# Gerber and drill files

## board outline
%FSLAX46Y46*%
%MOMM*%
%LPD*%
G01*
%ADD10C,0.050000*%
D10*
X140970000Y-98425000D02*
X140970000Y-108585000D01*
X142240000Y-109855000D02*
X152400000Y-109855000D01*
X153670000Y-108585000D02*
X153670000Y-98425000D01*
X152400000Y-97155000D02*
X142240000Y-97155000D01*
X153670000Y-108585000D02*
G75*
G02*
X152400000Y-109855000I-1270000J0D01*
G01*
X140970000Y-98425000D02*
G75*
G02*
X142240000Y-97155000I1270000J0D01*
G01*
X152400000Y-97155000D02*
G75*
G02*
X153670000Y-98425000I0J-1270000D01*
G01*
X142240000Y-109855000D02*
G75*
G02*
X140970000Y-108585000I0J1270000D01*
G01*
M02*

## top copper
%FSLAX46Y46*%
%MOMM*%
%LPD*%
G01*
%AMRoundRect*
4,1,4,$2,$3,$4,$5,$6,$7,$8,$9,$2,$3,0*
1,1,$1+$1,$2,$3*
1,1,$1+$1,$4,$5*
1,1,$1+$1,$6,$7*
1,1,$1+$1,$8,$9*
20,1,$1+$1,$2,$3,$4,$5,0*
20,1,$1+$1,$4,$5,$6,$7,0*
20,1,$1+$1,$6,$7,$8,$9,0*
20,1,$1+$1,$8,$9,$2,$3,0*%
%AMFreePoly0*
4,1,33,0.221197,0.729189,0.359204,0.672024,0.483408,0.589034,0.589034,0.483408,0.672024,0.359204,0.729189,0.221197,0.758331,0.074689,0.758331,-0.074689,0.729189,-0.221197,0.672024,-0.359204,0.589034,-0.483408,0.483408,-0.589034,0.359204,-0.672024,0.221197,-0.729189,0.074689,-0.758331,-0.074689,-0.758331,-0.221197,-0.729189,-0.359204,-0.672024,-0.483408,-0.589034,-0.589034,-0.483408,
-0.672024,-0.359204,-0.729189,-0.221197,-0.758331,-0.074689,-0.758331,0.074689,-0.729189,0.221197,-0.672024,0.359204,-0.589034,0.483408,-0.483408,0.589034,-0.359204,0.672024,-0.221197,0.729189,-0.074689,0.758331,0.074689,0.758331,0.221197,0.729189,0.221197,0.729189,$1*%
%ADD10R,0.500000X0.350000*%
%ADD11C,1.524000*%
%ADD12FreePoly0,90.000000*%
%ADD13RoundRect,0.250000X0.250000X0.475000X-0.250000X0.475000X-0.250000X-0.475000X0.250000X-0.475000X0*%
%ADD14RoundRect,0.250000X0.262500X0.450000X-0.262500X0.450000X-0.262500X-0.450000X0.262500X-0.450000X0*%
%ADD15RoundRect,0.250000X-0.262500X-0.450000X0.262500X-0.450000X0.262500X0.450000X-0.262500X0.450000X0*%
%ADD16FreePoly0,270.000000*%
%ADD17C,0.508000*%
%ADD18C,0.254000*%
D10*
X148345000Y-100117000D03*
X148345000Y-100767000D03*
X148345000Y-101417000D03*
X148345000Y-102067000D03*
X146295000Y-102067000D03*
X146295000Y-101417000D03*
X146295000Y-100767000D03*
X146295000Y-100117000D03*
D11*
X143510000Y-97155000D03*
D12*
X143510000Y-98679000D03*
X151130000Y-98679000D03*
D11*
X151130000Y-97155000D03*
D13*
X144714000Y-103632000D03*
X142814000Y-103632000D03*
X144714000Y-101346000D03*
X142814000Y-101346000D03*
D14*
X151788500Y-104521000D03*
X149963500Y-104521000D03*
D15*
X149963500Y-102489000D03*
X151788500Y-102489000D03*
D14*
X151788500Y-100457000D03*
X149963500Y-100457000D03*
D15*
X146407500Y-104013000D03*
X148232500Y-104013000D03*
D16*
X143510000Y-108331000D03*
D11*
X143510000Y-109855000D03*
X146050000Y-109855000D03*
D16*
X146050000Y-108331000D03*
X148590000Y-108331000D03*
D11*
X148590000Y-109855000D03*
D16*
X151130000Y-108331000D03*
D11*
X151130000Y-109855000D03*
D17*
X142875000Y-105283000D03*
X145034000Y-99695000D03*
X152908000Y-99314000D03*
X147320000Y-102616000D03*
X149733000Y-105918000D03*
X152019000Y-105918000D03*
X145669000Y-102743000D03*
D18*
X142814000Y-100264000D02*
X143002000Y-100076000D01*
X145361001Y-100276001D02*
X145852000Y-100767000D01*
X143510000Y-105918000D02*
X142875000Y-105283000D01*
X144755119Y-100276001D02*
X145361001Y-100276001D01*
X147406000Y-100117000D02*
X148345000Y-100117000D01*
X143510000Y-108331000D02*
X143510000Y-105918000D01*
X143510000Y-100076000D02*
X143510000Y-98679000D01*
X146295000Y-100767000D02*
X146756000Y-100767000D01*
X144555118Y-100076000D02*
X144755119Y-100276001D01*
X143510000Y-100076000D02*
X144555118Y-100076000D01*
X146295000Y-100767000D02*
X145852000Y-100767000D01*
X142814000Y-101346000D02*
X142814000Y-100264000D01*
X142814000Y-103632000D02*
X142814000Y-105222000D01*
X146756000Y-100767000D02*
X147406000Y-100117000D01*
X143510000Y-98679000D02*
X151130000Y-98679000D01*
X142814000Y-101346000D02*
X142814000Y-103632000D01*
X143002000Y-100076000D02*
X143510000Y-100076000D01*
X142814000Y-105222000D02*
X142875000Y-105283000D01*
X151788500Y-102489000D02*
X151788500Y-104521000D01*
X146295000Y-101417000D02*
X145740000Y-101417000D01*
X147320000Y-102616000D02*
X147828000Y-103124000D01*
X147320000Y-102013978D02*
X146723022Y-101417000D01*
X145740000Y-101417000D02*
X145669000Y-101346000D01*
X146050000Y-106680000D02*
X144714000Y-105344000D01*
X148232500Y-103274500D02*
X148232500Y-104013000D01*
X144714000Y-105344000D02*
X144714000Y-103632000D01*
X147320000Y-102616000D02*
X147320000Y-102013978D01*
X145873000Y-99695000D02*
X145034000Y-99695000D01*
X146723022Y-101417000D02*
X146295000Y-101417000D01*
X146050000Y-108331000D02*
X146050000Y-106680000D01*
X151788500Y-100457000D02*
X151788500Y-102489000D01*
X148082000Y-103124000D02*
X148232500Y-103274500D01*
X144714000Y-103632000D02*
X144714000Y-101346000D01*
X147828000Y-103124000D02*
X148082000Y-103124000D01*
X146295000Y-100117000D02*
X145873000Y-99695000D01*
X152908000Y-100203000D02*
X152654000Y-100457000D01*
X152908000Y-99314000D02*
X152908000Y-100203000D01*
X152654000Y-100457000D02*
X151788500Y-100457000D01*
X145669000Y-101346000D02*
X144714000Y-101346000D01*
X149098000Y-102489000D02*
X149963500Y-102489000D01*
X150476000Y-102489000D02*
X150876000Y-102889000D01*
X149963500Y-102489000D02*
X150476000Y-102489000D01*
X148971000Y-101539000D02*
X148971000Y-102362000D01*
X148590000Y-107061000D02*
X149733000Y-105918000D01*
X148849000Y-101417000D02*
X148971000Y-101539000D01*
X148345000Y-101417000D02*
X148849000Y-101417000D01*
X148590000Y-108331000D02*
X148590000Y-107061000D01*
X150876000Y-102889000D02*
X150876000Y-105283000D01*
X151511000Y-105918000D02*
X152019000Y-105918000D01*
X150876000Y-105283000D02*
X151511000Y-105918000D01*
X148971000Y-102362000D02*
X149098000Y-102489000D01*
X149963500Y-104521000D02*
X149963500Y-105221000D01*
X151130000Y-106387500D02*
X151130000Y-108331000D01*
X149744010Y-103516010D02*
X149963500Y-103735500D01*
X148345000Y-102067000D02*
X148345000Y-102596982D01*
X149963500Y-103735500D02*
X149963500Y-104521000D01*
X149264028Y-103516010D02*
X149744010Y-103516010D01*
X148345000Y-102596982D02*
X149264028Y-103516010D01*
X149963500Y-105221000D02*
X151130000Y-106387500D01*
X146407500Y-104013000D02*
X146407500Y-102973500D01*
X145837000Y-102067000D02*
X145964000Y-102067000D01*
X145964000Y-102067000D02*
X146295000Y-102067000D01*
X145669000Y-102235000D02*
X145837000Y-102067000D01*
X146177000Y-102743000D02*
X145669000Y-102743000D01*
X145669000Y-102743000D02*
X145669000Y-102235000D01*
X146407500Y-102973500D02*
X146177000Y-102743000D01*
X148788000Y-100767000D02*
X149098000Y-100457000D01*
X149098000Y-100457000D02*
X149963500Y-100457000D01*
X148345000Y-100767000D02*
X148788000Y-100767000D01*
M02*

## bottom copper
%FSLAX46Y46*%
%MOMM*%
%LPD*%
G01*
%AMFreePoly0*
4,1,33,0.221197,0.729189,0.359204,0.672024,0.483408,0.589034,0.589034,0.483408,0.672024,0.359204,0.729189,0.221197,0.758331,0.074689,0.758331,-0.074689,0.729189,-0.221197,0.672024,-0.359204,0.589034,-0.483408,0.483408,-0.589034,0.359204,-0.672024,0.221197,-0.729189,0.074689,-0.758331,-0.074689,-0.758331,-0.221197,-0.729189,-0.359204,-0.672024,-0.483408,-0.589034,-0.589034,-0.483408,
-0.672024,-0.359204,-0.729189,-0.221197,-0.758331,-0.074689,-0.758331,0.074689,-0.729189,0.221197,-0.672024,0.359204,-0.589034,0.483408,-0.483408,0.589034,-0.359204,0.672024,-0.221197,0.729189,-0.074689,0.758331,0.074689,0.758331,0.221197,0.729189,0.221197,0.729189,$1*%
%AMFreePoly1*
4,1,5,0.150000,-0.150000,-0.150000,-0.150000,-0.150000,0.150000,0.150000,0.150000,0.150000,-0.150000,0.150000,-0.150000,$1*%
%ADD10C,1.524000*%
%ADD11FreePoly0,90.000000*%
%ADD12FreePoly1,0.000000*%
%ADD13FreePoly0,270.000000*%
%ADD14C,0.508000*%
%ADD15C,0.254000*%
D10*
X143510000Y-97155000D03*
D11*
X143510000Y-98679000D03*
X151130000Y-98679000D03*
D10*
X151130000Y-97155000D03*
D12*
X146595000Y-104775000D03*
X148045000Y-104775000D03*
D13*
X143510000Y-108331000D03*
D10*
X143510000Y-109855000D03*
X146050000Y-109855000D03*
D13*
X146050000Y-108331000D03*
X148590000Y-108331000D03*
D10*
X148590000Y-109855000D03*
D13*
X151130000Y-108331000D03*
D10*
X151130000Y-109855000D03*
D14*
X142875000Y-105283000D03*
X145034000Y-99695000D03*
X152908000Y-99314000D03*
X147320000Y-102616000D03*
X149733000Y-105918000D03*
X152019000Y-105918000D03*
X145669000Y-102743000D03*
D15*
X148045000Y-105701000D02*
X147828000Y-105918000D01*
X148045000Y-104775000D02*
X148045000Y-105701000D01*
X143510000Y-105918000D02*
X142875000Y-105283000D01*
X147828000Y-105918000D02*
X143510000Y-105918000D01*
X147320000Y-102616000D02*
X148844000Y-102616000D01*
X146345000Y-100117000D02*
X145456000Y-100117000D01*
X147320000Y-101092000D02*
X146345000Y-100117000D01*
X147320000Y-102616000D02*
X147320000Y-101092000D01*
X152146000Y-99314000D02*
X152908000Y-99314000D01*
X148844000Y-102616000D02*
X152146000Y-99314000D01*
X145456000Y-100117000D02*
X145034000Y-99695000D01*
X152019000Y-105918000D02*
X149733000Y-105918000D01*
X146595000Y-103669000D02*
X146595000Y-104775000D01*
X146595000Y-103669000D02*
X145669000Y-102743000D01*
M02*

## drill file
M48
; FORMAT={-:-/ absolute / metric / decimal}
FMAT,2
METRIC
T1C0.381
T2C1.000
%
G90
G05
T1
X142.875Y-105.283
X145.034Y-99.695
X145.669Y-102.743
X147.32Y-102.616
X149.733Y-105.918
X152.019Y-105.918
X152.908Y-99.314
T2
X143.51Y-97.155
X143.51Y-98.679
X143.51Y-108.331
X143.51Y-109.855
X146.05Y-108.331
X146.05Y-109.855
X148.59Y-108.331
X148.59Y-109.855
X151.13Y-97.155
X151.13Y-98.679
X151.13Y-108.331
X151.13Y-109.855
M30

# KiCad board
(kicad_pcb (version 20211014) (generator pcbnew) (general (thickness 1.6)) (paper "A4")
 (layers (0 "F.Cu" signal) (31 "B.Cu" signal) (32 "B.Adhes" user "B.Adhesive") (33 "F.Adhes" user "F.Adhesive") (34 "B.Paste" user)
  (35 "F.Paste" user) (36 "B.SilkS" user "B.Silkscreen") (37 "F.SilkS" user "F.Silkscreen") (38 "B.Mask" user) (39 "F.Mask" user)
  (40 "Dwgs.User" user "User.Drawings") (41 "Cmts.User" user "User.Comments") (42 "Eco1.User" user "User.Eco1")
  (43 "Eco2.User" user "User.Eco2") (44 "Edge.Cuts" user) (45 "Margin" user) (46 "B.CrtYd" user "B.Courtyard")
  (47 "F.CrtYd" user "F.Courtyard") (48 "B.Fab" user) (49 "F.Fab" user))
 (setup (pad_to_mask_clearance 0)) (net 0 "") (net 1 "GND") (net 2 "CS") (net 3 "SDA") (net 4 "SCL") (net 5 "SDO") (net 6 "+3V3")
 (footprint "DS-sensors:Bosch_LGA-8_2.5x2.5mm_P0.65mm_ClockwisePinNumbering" (layer "F.Cu") (at 147.32 101.092 -90)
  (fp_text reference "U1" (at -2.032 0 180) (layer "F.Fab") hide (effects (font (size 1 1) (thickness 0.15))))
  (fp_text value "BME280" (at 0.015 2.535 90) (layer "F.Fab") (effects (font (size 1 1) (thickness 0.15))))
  (pad "1" smd rect locked (at -0.975 -1.025) (size 0.5 0.35) (layers "F.Cu" "F.Paste" "F.Mask") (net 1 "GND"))
  (pad "2" smd rect locked (at -0.325 -1.025) (size 0.5 0.35) (layers "F.Cu" "F.Paste" "F.Mask") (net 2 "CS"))
  (pad "3" smd rect locked (at 0.325 -1.025) (size 0.5 0.35) (layers "F.Cu" "F.Paste" "F.Mask") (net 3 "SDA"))
  (pad "4" smd rect locked (at 0.975 -1.025) (size 0.5 0.35) (layers "F.Cu" "F.Paste" "F.Mask") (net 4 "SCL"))
  (pad "5" smd rect locked (at 0.975 1.025) (size 0.5 0.35) (layers "F.Cu" "F.Paste" "F.Mask") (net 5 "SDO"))
  (pad "6" smd rect locked (at 0.325 1.025) (size 0.5 0.35) (layers "F.Cu" "F.Paste" "F.Mask") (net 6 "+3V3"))
  (pad "7" smd rect locked (at -0.325 1.025) (size 0.5 0.35) (layers "F.Cu" "F.Paste" "F.Mask") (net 1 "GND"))
  (pad "8" smd rect locked (at -0.975 1.025) (size 0.5 0.35) (layers "F.Cu" "F.Paste" "F.Mask") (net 6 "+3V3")))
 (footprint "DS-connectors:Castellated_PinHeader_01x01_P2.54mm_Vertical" (layer "F.Cu") (at 141.478 98.679 90)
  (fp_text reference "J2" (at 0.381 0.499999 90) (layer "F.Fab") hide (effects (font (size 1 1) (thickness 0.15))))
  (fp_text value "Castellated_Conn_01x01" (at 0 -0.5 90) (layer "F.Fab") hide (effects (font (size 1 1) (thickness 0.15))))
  (pad "1" thru_hole circle locked (at 1.524 2.032 90) (size 1.524 1.524) (drill 1) (layers *.Cu *.Mask) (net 1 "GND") (zone_connect 0))
  (pad "1" thru_hole custom locked (at 0 2.032 90) (size 1.524 1.524) (drill 1) (layers *.Cu *.Mask) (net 1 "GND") (zone_connect 0)
   (options (clearance outline) (anchor circle)) (primitives)))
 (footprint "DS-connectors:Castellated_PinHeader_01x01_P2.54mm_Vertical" (layer "F.Cu") (at 149.098 98.679 90)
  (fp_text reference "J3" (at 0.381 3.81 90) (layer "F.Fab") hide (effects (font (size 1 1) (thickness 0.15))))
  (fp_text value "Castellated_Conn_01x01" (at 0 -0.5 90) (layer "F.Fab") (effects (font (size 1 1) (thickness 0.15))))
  (pad "1" thru_hole custom locked (at 0 2.032 90) (size 1.524 1.524) (drill 1) (layers *.Cu *.Mask) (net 1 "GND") (zone_connect 0)
   (options (clearance outline) (anchor circle)) (primitives))
  (pad "1" thru_hole circle locked (at 1.524 2.032 90) (size 1.524 1.524) (drill 1) (layers *.Cu *.Mask) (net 1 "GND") (zone_connect 0)))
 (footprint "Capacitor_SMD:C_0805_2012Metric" (layer "F.Cu") (at 143.764 103.632 180)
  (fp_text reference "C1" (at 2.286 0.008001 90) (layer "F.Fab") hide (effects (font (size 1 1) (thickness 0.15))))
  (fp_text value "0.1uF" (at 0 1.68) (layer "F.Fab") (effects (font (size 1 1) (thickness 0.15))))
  (pad "1" smd roundrect locked (at -0.95 0 180) (size 1 1.45) (layers "F.Cu" "F.Paste" "F.Mask") (roundrect_rratio 0.25) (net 6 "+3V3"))
  (pad "2" smd roundrect locked (at 0.95 0 180) (size 1 1.45) (layers "F.Cu" "F.Paste" "F.Mask") (roundrect_rratio 0.25) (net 1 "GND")))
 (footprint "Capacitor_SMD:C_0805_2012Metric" (layer "F.Cu") (at 143.764 101.346 180)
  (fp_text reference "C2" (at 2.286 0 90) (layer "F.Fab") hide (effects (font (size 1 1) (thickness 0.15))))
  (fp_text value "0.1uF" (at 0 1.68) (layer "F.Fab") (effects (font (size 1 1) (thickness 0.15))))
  (pad "1" smd roundrect locked (at -0.95 0 180) (size 1 1.45) (layers "F.Cu" "F.Paste" "F.Mask") (roundrect_rratio 0.25) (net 6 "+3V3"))
  (pad "2" smd roundrect locked (at 0.95 0 180) (size 1 1.45) (layers "F.Cu" "F.Paste" "F.Mask") (roundrect_rratio 0.25) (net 1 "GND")))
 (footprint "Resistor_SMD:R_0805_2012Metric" (layer "F.Cu") (at 150.876 104.521 180)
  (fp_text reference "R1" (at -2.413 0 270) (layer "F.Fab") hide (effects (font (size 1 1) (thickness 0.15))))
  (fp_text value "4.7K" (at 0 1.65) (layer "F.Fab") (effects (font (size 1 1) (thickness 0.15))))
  (pad "1" smd roundrect locked (at -0.9125 0 180) (size 1.025 1.4) (layers "F.Cu" "F.Paste" "F.Mask") (roundrect_rratio 0.243902)
   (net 6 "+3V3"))
  (pad "2" smd roundrect locked (at 0.9125 0 180) (size 1.025 1.4) (layers "F.Cu" "F.Paste" "F.Mask") (roundrect_rratio 0.243902)
   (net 4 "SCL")))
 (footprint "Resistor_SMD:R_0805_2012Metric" (layer "F.Cu") (at 150.876 102.489)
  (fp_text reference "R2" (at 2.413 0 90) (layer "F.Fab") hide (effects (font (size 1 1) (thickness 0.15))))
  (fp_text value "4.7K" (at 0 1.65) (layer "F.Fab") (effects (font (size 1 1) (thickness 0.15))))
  (pad "1" smd roundrect locked (at -0.9125 0) (size 1.025 1.4) (layers "F.Cu" "F.Paste" "F.Mask") (roundrect_rratio 0.243902) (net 3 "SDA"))
  (pad "2" smd roundrect locked (at 0.9125 0) (size 1.025 1.4) (layers "F.Cu" "F.Paste" "F.Mask") (roundrect_rratio 0.243902) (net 6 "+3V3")))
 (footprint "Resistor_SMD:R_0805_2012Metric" (layer "F.Cu") (at 150.876 100.457 180)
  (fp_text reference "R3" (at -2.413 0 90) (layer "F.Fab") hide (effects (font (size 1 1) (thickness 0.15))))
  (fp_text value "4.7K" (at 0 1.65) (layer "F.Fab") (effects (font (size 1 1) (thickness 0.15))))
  (pad "1" smd roundrect locked (at -0.9125 0 180) (size 1.025 1.4) (layers "F.Cu" "F.Paste" "F.Mask") (roundrect_rratio 0.243902)
   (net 6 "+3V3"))
  (pad "2" smd roundrect locked (at 0.9125 0 180) (size 1.025 1.4) (layers "F.Cu" "F.Paste" "F.Mask") (roundrect_rratio 0.243902)
   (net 2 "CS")))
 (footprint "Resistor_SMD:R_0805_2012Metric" (layer "F.Cu") (at 147.32 104.013)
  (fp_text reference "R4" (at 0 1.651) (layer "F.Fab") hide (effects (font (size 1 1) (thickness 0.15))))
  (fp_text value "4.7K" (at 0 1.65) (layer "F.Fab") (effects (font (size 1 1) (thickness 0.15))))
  (pad "1" smd roundrect locked (at -0.9125 0) (size 1.025 1.4) (layers "F.Cu" "F.Paste" "F.Mask") (roundrect_rratio 0.243902) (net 5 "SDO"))
  (pad "2" smd roundrect locked (at 0.9125 0) (size 1.025 1.4) (layers "F.Cu" "F.Paste" "F.Mask") (roundrect_rratio 0.243902) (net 6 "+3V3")))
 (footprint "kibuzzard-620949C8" (layer "F.Cu") (at 143.51 105.537 90)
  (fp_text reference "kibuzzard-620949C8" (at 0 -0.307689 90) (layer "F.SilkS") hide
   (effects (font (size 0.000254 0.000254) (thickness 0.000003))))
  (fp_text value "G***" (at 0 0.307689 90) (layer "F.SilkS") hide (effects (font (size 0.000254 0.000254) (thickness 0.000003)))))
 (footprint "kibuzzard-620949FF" (layer "F.Cu") (at 151.13 107.061 90)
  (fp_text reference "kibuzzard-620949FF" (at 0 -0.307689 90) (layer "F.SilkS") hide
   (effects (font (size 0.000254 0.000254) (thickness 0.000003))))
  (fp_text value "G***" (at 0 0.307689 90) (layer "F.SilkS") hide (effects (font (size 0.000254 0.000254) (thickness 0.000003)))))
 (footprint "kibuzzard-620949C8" (layer "F.Cu") (at 148.59 106.299 90)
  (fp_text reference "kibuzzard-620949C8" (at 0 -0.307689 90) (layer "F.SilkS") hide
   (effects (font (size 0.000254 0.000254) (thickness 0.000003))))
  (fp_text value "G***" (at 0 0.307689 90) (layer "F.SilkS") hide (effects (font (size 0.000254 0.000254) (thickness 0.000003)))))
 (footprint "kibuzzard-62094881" (layer "F.Cu") (at 148.717 97.917)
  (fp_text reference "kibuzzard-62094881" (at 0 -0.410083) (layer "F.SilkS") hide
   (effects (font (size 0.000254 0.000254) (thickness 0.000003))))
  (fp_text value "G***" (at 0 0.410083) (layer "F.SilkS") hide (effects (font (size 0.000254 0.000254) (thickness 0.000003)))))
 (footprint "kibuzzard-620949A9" (layer "F.Cu") (at 143.51 107.061 90)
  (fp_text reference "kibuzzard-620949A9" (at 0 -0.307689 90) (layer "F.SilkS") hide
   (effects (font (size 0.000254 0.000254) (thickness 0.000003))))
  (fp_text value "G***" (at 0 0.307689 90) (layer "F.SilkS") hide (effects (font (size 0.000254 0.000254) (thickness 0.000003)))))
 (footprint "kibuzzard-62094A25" (layer "F.Cu") (at 151.13 106.299 90)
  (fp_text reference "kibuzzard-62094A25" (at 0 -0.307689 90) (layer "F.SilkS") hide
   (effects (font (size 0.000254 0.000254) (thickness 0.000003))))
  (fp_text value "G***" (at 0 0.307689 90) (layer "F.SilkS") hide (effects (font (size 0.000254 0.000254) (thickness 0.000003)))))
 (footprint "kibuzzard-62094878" (layer "F.Cu") (at 147.7772 97.917)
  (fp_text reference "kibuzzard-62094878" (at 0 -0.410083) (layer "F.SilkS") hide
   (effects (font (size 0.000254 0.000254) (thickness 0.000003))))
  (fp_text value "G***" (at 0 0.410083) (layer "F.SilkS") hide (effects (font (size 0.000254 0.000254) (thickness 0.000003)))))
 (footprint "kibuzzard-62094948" (layer "F.Cu") (at 147.32 98.933)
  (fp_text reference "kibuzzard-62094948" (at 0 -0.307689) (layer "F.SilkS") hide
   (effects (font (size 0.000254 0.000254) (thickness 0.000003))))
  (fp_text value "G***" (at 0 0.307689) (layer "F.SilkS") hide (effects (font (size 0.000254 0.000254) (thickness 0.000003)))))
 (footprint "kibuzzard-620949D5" (layer "F.Cu") (at 146.05 105.537 90)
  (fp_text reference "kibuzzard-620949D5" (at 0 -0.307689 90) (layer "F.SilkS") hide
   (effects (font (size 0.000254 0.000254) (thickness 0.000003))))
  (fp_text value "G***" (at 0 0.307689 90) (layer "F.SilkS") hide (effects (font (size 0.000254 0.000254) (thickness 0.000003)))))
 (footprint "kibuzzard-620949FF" (layer "F.Cu") (at 148.59 107.061 90)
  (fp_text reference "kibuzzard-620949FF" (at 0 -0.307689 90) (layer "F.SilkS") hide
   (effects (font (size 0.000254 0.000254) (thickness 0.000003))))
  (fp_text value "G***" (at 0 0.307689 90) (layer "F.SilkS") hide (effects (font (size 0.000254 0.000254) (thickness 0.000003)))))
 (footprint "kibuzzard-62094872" (layer "F.Cu") (at 146.9136 97.917)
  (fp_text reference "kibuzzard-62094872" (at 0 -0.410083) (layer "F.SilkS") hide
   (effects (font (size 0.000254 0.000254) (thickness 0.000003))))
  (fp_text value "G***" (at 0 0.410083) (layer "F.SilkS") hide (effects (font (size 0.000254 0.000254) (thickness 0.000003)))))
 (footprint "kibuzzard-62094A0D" (layer "F.Cu") (at 148.59 105.537 90)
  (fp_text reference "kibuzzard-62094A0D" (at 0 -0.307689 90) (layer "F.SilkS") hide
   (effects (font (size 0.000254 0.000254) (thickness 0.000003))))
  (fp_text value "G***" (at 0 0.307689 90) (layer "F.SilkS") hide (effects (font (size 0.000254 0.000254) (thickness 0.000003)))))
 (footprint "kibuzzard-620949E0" (layer "F.Cu") (at 146.05 106.299 90)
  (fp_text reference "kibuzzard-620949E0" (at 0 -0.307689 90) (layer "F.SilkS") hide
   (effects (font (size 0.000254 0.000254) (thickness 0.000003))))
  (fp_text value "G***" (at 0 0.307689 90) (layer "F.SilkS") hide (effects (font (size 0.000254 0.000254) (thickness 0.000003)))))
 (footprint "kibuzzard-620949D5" (layer "F.Cu") (at 146.05 107.061 90)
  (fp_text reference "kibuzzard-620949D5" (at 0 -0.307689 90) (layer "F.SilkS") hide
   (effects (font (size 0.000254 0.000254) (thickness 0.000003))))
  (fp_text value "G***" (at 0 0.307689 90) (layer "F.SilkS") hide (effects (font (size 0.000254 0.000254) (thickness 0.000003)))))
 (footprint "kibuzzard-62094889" (layer "F.Cu") (at 149.6568 97.917)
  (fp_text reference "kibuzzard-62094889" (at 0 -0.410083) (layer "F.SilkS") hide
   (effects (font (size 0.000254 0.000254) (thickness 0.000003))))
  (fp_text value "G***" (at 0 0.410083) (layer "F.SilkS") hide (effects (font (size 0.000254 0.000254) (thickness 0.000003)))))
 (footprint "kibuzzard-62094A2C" (layer "F.Cu") (at 151.13 105.537 90)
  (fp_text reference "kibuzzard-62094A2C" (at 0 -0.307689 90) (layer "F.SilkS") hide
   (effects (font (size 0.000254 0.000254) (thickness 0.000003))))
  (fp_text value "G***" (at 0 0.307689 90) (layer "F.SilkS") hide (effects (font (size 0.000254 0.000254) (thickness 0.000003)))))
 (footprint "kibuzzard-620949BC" (layer "F.Cu") (at 143.51 106.299 90)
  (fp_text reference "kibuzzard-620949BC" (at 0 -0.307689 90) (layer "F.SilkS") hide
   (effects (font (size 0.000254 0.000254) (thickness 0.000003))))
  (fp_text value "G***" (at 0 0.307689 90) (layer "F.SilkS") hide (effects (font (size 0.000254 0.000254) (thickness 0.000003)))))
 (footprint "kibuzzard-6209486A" (layer "F.Cu") (at 145.9484 97.917)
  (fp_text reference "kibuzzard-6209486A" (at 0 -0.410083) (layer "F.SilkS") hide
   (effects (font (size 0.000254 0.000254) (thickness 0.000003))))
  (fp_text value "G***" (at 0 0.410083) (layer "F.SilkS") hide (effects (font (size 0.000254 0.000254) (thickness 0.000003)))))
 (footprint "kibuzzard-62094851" (layer "F.Cu") (at 144.9324 97.917)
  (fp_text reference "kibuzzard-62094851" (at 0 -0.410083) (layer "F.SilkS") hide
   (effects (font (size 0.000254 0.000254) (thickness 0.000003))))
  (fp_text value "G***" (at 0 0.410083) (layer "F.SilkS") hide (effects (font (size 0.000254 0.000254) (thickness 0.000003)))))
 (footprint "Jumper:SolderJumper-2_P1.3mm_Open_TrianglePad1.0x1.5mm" (layer "B.Cu") (at 147.32 104.775)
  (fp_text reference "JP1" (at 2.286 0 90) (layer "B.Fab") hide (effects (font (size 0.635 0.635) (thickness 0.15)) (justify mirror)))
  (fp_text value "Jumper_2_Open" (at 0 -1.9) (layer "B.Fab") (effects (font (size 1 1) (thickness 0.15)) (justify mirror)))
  (pad "1" smd custom locked (at -0.725 0) (size 0.3 0.3) (layers "B.Cu" "B.Mask") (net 5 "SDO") (zone_connect 2)
   (options (clearance outline) (anchor rect)) (primitives))
  (pad "2" smd custom locked (at 0.725 0) (size 0.3 0.3) (layers "B.Cu" "B.Mask") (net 1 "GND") (zone_connect 2)
   (options (clearance outline) (anchor rect)) (primitives)))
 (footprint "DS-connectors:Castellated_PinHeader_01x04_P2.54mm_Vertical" (layer "B.Cu") (at 140.97 108.331 -90)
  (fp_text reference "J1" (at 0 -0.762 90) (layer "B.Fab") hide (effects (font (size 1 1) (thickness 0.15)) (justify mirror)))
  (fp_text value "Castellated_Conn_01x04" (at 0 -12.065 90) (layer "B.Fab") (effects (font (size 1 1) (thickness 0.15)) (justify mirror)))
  (pad "1" thru_hole custom locked (at 0 -2.54 270) (size 1.524 1.524) (drill 1) (layers *.Cu *.Mask) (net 1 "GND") (zone_connect 0)
   (options (clearance outline) (anchor circle)) (primitives))
  (pad "1" thru_hole circle locked (at 1.524 -2.54 270) (size 1.524 1.524) (drill 1) (layers *.Cu *.Mask) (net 1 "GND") (zone_connect 0))
  (pad "2" thru_hole circle locked (at 1.524 -5.08 270) (size 1.524 1.524) (drill 1) (layers *.Cu *.Mask) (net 6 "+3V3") (zone_connect 0))
  (pad "2" thru_hole custom locked (at 0 -5.08 270) (size 1.524 1.524) (drill 1) (layers *.Cu *.Mask) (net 6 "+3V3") (zone_connect 0)
   (options (clearance outline) (anchor circle)) (primitives))
  (pad "3" thru_hole custom locked (at 0 -7.62 270) (size 1.524 1.524) (drill 1) (layers *.Cu *.Mask) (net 3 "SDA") (zone_connect 0)
   (options (clearance outline) (anchor circle)) (primitives))
  (pad "3" thru_hole circle locked (at 1.524 -7.62 270) (size 1.524 1.524) (drill 1) (layers *.Cu *.Mask) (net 3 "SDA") (zone_connect 0))
  (pad "4" thru_hole custom locked (at 0 -10.16 270) (size 1.524 1.524) (drill 1) (layers *.Cu *.Mask) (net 4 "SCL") (zone_connect 0)
   (options (clearance outline) (anchor circle)) (primitives))
  (pad "4" thru_hole circle locked (at 1.524 -10.16 270) (size 1.524 1.524) (drill 1) (layers *.Cu *.Mask) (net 4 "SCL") (zone_connect 0)))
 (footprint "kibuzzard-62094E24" (layer "B.Cu") (at 144.1704 99.4664 180)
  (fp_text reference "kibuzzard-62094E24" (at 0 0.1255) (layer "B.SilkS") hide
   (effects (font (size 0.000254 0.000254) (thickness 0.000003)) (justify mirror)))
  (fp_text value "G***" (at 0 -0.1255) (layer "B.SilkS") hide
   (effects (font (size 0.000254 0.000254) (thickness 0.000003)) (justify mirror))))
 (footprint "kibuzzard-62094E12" (layer "B.Cu") (at 148.8948 99.1108 180)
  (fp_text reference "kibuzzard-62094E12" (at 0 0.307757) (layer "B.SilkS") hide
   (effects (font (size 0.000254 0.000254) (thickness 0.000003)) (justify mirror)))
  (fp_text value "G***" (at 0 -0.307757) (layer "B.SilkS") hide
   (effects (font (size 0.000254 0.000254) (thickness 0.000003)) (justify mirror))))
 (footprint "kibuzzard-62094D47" (layer "B.Cu") (at 147.32 101.854 180)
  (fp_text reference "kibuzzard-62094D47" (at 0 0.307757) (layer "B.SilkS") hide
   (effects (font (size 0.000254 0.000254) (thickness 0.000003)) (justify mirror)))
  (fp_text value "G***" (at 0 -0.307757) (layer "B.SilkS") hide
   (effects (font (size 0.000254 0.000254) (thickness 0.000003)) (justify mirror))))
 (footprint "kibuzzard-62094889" (layer "B.Cu") (at 144.9578 98.044 180)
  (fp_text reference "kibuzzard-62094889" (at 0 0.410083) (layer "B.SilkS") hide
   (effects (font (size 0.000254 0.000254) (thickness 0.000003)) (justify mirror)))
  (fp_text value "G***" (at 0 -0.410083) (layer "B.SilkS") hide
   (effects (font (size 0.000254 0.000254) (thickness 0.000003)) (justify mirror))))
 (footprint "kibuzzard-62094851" (layer "B.Cu") (at 149.6822 98.044 180)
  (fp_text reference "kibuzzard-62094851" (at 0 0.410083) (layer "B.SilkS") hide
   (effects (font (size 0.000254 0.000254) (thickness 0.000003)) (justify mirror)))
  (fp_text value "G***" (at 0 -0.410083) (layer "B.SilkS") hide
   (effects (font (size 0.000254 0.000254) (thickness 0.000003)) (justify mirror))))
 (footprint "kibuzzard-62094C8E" (layer "B.Cu") (at 147.32 99.949 180)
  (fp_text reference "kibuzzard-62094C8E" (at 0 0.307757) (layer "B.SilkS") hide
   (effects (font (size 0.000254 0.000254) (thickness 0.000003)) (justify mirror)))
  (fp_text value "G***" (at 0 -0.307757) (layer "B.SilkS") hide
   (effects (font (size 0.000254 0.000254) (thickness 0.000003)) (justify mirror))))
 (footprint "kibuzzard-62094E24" (layer "B.Cu") (at 147.32 99.4156 180)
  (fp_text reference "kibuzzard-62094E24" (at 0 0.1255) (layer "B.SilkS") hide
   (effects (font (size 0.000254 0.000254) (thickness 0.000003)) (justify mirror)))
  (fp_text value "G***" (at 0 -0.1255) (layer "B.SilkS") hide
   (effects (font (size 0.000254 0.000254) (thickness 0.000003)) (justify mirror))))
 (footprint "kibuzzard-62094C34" (layer "B.Cu") (at 145.6944 99.1108 180)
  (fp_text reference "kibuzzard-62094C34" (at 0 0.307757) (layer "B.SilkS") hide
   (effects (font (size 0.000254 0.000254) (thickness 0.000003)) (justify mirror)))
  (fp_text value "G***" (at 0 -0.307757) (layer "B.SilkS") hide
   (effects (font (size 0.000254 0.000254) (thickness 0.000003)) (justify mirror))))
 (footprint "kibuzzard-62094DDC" (layer "B.Cu") (at 141.732 103.505 -90)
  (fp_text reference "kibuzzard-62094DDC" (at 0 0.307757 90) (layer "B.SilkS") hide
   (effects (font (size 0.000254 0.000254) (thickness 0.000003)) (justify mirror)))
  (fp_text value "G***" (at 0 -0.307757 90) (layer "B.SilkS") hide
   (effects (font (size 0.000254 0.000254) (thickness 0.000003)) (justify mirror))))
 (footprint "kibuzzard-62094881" (layer "B.Cu") (at 145.8976 98.044 180)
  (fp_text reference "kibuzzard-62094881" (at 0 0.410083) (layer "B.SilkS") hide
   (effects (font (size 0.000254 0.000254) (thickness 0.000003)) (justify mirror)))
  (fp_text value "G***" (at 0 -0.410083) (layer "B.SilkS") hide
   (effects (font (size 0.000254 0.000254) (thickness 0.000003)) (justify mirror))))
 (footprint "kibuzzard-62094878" (layer "B.Cu") (at 146.8374 98.044 180)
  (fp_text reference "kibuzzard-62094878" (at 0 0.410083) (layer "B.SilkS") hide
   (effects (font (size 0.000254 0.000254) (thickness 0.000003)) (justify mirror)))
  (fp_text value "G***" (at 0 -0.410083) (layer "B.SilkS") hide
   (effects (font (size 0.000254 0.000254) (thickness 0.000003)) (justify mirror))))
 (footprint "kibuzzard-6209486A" (layer "B.Cu") (at 148.6662 98.044 180)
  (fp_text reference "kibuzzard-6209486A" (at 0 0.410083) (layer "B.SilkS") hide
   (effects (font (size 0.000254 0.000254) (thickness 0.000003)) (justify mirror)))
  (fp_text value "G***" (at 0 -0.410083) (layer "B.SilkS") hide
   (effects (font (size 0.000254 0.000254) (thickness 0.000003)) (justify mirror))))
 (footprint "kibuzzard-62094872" (layer "B.Cu") (at 147.701 98.044 180)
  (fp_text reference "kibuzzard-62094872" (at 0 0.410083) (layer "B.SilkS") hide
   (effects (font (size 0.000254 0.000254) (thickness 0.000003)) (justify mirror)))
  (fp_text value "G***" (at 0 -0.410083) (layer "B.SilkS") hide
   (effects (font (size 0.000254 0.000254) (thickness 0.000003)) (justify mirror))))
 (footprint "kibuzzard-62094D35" (layer "B.Cu") (at 147.32 100.965 180)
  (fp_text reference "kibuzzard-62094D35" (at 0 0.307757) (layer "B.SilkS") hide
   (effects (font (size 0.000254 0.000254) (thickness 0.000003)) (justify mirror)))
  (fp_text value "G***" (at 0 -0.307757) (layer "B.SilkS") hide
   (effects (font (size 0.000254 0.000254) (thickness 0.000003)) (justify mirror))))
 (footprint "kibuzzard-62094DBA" (layer "B.Cu") (at 147.32 106.299 180)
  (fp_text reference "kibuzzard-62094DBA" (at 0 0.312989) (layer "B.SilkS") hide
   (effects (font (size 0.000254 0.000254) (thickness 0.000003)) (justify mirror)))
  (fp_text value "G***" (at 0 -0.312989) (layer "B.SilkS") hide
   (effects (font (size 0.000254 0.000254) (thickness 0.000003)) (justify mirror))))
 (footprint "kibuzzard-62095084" (layer "B.Cu") (at 147.32 103.251 180)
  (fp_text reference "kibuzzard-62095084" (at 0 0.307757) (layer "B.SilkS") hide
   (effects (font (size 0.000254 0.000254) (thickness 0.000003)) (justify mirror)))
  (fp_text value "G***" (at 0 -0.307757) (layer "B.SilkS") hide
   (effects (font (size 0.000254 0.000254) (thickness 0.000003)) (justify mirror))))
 (gr_line (start 140.97 98.425) (end 140.97 108.585) (layer "Edge.Cuts") (width 0.05))
 (gr_line (start 142.24 109.855) (end 152.4 109.855) (layer "Edge.Cuts") (width 0.05))
 (gr_line (start 153.67 108.585) (end 153.67 98.425) (layer "Edge.Cuts") (width 0.05))
 (gr_line (start 152.4 97.155) (end 142.24 97.155) (layer "Edge.Cuts") (width 0.05))
 (gr_arc (start 153.67 108.585) (mid 153.298026 109.483026) (end 152.4 109.855) (layer "Edge.Cuts") (width 0.05))
 (gr_arc (start 140.97 98.425) (mid 141.341974 97.526974) (end 142.24 97.155) (layer "Edge.Cuts") (width 0.05))
 (gr_arc (start 152.4 97.155) (mid 153.298026 97.526974) (end 153.67 98.425) (layer "Edge.Cuts") (width 0.05))
 (gr_arc (start 142.24 109.855) (mid 141.341974 109.483026) (end 140.97 108.585) (layer "Edge.Cuts") (width 0.05))
 (segment (start 142.814 100.264) (end 143.002 100.076) (width 0.254) (layer "F.Cu") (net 1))
 (segment (start 145.361001 100.276001) (end 145.852 100.767) (width 0.254) (layer "F.Cu") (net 1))
 (segment (start 143.51 105.918) (end 142.875 105.283) (width 0.254) (layer "F.Cu") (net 1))
 (segment (start 144.755119 100.276001) (end 145.361001 100.276001) (width 0.254) (layer "F.Cu") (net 1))
 (segment (start 147.406 100.117) (end 148.345 100.117) (width 0.254) (layer "F.Cu") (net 1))
 (segment (start 143.51 108.331) (end 143.51 105.918) (width 0.254) (layer "F.Cu") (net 1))
 (segment (start 143.51 100.076) (end 143.51 98.679) (width 0.254) (layer "F.Cu") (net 1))
 (segment (start 146.295 100.767) (end 146.756 100.767) (width 0.254) (layer "F.Cu") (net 1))
 (segment (start 144.555118 100.076) (end 144.755119 100.276001) (width 0.254) (layer "F.Cu") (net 1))
 (segment (start 143.51 100.076) (end 144.555118 100.076) (width 0.254) (layer "F.Cu") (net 1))
 (segment (start 146.295 100.767) (end 145.852 100.767) (width 0.254) (layer "F.Cu") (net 1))
 (segment (start 142.814 101.346) (end 142.814 100.264) (width 0.254) (layer "F.Cu") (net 1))
 (segment (start 142.814 103.632) (end 142.814 105.222) (width 0.254) (layer "F.Cu") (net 1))
 (segment (start 146.756 100.767) (end 147.406 100.117) (width 0.254) (layer "F.Cu") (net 1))
 (segment (start 143.51 98.679) (end 151.13 98.679) (width 0.254) (layer "F.Cu") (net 1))
 (segment (start 142.814 101.346) (end 142.814 103.632) (width 0.254) (layer "F.Cu") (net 1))
 (segment (start 143.002 100.076) (end 143.51 100.076) (width 0.254) (layer "F.Cu") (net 1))
 (segment (start 142.814 105.222) (end 142.875 105.283) (width 0.254) (layer "F.Cu") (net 1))
 (via (at 142.875 105.283) (size 0.508) (drill 0.381) (layers "F.Cu" "B.Cu") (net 1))
 (segment (start 148.045 105.701) (end 147.828 105.918) (width 0.254) (layer "B.Cu") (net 1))
 (segment (start 148.045 104.775) (end 148.045 105.701) (width 0.254) (layer "B.Cu") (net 1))
 (segment (start 143.51 105.918) (end 142.875 105.283) (width 0.254) (layer "B.Cu") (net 1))
 (segment (start 147.828 105.918) (end 143.51 105.918) (width 0.254) (layer "B.Cu") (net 1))
 (segment (start 151.7885 102.489) (end 151.7885 104.521) (width 0.254) (layer "F.Cu") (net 6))
 (segment (start 146.295 101.417) (end 145.74 101.417) (width 0.254) (layer "F.Cu") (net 6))
 (segment (start 147.32 102.616) (end 147.828 103.124) (width 0.254) (layer "F.Cu") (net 6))
 (segment (start 147.32 102.013978) (end 146.723022 101.417) (width 0.254) (layer "F.Cu") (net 6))
 (segment (start 145.74 101.417) (end 145.669 101.346) (width 0.254) (layer "F.Cu") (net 6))
 (segment (start 146.05 106.68) (end 144.714 105.344) (width 0.254) (layer "F.Cu") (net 6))
 (segment (start 148.2325 103.2745) (end 148.2325 104.013) (width 0.254) (layer "F.Cu") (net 6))
 (segment (start 144.714 105.344) (end 144.714 103.632) (width 0.254) (layer "F.Cu") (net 6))
 (segment (start 147.32 102.616) (end 147.32 102.013978) (width 0.254) (layer "F.Cu") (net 6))
 (segment (start 145.873 99.695) (end 145.034 99.695) (width 0.254) (layer "F.Cu") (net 6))
 (segment (start 146.723022 101.417) (end 146.295 101.417) (width 0.254) (layer "F.Cu") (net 6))
 (segment (start 146.05 108.331) (end 146.05 106.68) (width 0.254) (layer "F.Cu") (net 6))
 (segment (start 151.7885 100.457) (end 151.7885 102.489) (width 0.254) (layer "F.Cu") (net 6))
 (segment (start 148.082 103.124) (end 148.2325 103.2745) (width 0.254) (layer "F.Cu") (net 6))
 (segment (start 144.714 103.632) (end 144.714 101.346) (width 0.254) (layer "F.Cu") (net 6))
 (segment (start 147.828 103.124) (end 148.082 103.124) (width 0.254) (layer "F.Cu") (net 6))
 (segment (start 146.295 100.117) (end 145.873 99.695) (width 0.254) (layer "F.Cu") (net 6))
 (segment (start 152.908 100.203) (end 152.654 100.457) (width 0.254) (layer "F.Cu") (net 6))
 (segment (start 152.908 99.314) (end 152.908 100.203) (width 0.254) (layer "F.Cu") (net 6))
 (segment (start 152.654 100.457) (end 151.7885 100.457) (width 0.254) (layer "F.Cu") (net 6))
 (segment (start 145.669 101.346) (end 144.714 101.346) (width 0.254) (layer "F.Cu") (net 6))
 (via (at 145.034 99.695) (size 0.508) (drill 0.381) (layers "F.Cu" "B.Cu") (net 6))
 (via (at 152.908 99.314) (size 0.508) (drill 0.381) (layers "F.Cu" "B.Cu") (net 6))
 (via (at 147.32 102.616) (size 0.508) (drill 0.381) (layers "F.Cu" "B.Cu") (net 6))
 (segment (start 147.32 102.616) (end 148.844 102.616) (width 0.254) (layer "B.Cu") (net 6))
 (segment (start 146.345 100.117) (end 145.456 100.117) (width 0.254) (layer "B.Cu") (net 6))
 (segment (start 147.32 101.092) (end 146.345 100.117) (width 0.254) (layer "B.Cu") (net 6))
 (segment (start 147.32 102.616) (end 147.32 101.092) (width 0.254) (layer "B.Cu") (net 6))
 (segment (start 152.146 99.314) (end 152.908 99.314) (width 0.254) (layer "B.Cu") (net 6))
 (segment (start 148.844 102.616) (end 152.146 99.314) (width 0.254) (layer "B.Cu") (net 6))
 (segment (start 145.456 100.117) (end 145.034 99.695) (width 0.254) (layer "B.Cu") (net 6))
 (segment (start 149.098 102.489) (end 149.9635 102.489) (width 0.254) (layer "F.Cu") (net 3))
 (segment (start 150.476 102.489) (end 150.876 102.889) (width 0.254) (layer "F.Cu") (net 3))
 (segment (start 149.9635 102.489) (end 150.476 102.489) (width 0.254) (layer "F.Cu") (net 3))
 (segment (start 148.971 101.539) (end 148.971 102.362) (width 0.254) (layer "F.Cu") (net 3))
 (segment (start 148.59 107.061) (end 149.733 105.918) (width 0.254) (layer "F.Cu") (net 3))
 (segment (start 148.849 101.417) (end 148.971 101.539) (width 0.254) (layer "F.Cu") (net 3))
 (segment (start 148.345 101.417) (end 148.849 101.417) (width 0.254) (layer "F.Cu") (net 3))
 (segment (start 148.59 108.331) (end 148.59 107.061) (width 0.254) (layer "F.Cu") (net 3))
 (segment (start 150.876 102.889) (end 150.876 105.283) (width 0.254) (layer "F.Cu") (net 3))
 (segment (start 151.511 105.918) (end 152.019 105.918) (width 0.254) (layer "F.Cu") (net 3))
 (segment (start 150.876 105.283) (end 151.511 105.918) (width 0.254) (layer "F.Cu") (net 3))
 (segment (start 148.971 102.362) (end 149.098 102.489) (width 0.254) (layer "F.Cu") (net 3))
 (via (at 149.733 105.918) (size 0.508) (drill 0.381) (layers "F.Cu" "B.Cu") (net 3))
 (via (at 152.019 105.918) (size 0.508) (drill 0.381) (layers "F.Cu" "B.Cu") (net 3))
 (segment (start 152.019 105.918) (end 149.733 105.918) (width 0.254) (layer "B.Cu") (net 3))
 (segment (start 149.9635 104.521) (end 149.9635 105.221) (width 0.254) (layer "F.Cu") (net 4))
 (segment (start 151.13 106.3875) (end 151.13 108.331) (width 0.254) (layer "F.Cu") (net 4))
 (segment (start 149.74401 103.51601) (end 149.9635 103.7355) (width 0.254) (layer "F.Cu") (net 4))
 (segment (start 148.345 102.067) (end 148.345 102.596982) (width 0.254) (layer "F.Cu") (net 4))
 (segment (start 149.9635 103.7355) (end 149.9635 104.521) (width 0.254) (layer "F.Cu") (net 4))
 (segment (start 149.264028 103.51601) (end 149.74401 103.51601) (width 0.254) (layer "F.Cu") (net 4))
 (segment (start 148.345 102.596982) (end 149.264028 103.51601) (width 0.254) (layer "F.Cu") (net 4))
 (segment (start 149.9635 105.221) (end 151.13 106.3875) (width 0.254) (layer "F.Cu") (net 4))
 (segment (start 146.4075 104.013) (end 146.4075 102.9735) (width 0.254) (layer "F.Cu") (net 5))
 (segment (start 145.837 102.067) (end 145.964 102.067) (width 0.254) (layer "F.Cu") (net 5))
 (segment (start 145.964 102.067) (end 146.295 102.067) (width 0.254) (layer "F.Cu") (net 5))
 (segment (start 145.669 102.235) (end 145.837 102.067) (width 0.254) (layer "F.Cu") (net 5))
 (segment (start 146.177 102.743) (end 145.669 102.743) (width 0.254) (layer "F.Cu") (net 5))
 (segment (start 145.669 102.743) (end 145.669 102.235) (width 0.254) (layer "F.Cu") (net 5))
 (segment (start 146.4075 102.9735) (end 146.177 102.743) (width 0.254) (layer "F.Cu") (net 5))
 (via (at 145.669 102.743) (size 0.508) (drill 0.381) (layers "F.Cu" "B.Cu") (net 5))
 (segment (start 146.595 103.669) (end 146.595 104.775) (width 0.254) (layer "B.Cu") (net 5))
 (segment (start 146.595 103.669) (end 145.669 102.743) (width 0.254) (layer "B.Cu") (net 5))
 (segment (start 148.788 100.767) (end 149.098 100.457) (width 0.254) (layer "F.Cu") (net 2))
 (segment (start 149.098 100.457) (end 149.9635 100.457) (width 0.254) (layer "F.Cu") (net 2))
 (segment (start 148.345 100.767) (end 148.788 100.767) (width 0.254) (layer "F.Cu") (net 2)))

